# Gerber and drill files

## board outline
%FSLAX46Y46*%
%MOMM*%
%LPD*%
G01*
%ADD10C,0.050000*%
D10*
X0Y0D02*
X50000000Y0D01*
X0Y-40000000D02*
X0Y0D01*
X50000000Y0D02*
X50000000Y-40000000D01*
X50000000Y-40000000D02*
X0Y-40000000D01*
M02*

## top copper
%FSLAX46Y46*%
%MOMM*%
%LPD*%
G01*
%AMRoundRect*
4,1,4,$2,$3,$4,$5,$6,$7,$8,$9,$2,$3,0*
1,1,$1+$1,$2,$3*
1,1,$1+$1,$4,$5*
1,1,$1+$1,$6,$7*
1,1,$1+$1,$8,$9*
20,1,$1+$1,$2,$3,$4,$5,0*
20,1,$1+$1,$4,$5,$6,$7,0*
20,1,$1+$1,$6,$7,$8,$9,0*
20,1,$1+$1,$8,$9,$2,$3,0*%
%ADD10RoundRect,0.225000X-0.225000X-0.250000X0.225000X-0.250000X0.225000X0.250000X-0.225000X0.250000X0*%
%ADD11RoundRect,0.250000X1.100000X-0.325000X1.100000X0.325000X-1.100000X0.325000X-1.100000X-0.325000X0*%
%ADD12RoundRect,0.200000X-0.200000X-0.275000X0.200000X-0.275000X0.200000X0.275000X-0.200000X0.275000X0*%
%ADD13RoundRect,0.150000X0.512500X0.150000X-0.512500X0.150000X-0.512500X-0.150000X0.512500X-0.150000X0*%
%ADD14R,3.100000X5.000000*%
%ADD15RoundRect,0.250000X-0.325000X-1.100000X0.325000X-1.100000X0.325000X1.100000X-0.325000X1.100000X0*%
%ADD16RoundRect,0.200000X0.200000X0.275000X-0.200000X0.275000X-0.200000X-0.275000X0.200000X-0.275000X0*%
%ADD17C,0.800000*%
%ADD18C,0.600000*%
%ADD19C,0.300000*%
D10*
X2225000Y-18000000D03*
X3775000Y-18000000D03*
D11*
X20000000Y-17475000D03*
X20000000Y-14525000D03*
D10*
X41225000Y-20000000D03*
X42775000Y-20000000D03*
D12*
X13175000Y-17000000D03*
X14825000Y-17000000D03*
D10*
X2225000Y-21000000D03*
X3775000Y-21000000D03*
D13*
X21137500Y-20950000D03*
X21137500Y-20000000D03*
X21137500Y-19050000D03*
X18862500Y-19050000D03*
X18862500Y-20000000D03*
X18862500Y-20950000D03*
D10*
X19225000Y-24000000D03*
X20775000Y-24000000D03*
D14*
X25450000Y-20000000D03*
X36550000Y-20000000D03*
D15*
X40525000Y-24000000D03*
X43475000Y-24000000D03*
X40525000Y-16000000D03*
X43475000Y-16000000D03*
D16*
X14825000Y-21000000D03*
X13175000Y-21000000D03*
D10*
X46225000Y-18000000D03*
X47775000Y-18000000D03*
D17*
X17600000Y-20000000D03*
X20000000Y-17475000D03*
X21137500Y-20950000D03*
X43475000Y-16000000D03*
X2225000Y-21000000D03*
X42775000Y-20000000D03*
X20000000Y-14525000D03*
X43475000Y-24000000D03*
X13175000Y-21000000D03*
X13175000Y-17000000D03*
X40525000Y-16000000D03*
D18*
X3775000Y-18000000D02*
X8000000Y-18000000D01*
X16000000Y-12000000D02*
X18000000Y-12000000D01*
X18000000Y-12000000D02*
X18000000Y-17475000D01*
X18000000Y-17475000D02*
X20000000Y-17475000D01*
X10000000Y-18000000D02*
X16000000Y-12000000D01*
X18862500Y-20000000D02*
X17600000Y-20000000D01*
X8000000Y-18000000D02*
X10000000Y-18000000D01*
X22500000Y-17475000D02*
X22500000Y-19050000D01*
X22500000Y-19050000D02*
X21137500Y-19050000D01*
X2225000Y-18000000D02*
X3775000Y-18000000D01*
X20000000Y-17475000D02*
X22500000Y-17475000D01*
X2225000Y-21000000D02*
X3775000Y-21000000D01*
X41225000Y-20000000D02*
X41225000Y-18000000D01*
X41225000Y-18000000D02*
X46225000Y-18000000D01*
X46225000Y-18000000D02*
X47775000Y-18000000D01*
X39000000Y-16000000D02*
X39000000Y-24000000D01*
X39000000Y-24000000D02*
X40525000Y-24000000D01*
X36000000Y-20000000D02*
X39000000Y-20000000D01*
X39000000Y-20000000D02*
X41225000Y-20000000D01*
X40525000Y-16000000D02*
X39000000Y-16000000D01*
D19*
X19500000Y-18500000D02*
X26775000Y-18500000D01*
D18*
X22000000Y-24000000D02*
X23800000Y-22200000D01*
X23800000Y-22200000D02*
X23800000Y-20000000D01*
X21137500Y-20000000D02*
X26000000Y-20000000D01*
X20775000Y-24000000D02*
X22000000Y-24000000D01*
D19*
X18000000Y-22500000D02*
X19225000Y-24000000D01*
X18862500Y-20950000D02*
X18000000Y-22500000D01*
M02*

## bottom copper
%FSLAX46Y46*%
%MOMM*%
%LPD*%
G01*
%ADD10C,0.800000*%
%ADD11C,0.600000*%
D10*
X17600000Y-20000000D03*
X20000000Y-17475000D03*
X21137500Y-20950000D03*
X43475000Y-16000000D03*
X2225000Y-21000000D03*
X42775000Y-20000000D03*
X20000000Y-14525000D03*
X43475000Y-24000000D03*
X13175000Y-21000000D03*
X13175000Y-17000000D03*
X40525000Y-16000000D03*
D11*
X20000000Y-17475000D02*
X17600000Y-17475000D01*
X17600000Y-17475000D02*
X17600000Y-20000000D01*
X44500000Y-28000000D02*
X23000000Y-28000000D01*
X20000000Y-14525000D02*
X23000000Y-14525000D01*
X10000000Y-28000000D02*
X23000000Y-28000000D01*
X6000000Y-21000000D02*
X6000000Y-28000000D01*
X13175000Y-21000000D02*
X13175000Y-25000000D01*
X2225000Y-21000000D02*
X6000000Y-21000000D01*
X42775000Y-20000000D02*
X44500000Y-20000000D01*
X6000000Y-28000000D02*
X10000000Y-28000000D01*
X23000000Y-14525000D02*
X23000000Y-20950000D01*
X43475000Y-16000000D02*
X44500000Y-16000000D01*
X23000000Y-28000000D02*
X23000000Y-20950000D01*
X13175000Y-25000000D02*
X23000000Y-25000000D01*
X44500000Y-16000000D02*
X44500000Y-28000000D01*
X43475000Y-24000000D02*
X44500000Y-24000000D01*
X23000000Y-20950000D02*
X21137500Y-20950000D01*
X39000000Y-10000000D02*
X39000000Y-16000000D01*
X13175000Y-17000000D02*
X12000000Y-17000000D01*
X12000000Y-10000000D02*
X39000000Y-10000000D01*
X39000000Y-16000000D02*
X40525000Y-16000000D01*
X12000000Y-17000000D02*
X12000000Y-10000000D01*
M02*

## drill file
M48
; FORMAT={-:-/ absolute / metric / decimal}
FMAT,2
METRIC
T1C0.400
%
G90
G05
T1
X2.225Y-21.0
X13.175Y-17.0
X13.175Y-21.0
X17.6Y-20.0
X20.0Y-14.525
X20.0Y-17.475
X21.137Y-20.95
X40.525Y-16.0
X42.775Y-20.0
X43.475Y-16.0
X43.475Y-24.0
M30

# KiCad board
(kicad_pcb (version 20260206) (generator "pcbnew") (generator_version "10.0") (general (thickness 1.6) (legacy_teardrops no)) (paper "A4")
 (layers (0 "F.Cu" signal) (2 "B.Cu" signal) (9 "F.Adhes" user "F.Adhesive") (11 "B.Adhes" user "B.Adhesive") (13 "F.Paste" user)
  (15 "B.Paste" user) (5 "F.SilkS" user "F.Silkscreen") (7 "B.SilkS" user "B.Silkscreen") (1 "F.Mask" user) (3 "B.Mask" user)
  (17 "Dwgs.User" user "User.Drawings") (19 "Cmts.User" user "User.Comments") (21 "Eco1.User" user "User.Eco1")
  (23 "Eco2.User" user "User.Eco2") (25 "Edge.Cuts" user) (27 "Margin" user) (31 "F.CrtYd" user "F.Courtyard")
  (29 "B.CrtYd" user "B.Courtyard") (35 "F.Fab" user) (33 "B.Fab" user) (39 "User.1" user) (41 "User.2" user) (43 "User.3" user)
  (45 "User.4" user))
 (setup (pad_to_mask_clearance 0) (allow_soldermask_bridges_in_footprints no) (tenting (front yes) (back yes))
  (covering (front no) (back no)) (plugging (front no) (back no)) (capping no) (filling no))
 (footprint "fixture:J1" (layer "F.Cu") (at 3 18)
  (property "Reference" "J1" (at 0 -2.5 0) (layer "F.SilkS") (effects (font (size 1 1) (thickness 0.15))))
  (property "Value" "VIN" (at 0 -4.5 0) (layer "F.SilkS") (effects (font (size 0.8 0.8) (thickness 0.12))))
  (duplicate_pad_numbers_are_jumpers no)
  (pad "1" smd roundrect (at -0.775 0) (size 0.9 0.95) (layers "F.Cu" "F.Mask" "F.Paste") (roundrect_rratio 0.25) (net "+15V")
   (thermal_bridge_angle 45))
  (pad "2" smd roundrect (at 0.775 0) (size 0.9 0.95) (layers "F.Cu" "F.Mask" "F.Paste") (roundrect_rratio 0.25) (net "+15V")
   (thermal_bridge_angle 45)))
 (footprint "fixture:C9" (layer "F.Cu") (at 20 16 90)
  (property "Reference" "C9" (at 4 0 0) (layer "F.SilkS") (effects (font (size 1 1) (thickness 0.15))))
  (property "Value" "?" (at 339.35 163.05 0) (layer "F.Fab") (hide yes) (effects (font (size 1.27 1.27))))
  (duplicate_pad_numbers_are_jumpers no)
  (pad "1" smd roundrect (at -1.475 0 90) (size 1.15 2.7) (layers "F.Cu" "F.Mask" "F.Paste") (roundrect_rratio 0.217391) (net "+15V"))
  (pad "2" smd roundrect (at 1.475 0 90) (size 1.15 2.7) (layers "F.Cu" "F.Mask" "F.Paste") (roundrect_rratio 0.217391) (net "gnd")))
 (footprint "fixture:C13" (layer "F.Cu") (at 42 20)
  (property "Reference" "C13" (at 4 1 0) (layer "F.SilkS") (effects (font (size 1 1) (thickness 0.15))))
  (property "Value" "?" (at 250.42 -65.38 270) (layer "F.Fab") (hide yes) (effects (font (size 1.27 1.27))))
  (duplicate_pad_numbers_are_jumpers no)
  (pad "1" smd roundrect (at -0.775 0) (size 0.9 0.95) (layers "F.Cu" "F.Mask" "F.Paste") (roundrect_rratio 0.25) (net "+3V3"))
  (pad "2" smd roundrect (at 0.775 0) (size 0.9 0.95) (layers "F.Cu" "F.Mask" "F.Paste") (roundrect_rratio 0.25) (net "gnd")))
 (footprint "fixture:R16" (layer "F.Cu") (at 14 17)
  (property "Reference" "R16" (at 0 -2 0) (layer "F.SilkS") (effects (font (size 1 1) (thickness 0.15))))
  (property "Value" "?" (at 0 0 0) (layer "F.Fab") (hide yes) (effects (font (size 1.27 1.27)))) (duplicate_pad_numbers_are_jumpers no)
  (pad "1" smd roundrect (at -0.825 0) (size 0.8 0.95) (layers "F.Cu" "F.Mask" "F.Paste") (roundrect_rratio 0.25) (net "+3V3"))
  (pad "2" smd roundrect (at 0.825 0) (size 0.8 0.95) (layers "F.Cu" "F.Mask" "F.Paste") (roundrect_rratio 0.25) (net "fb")))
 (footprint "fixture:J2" (layer "F.Cu") (at 3 21)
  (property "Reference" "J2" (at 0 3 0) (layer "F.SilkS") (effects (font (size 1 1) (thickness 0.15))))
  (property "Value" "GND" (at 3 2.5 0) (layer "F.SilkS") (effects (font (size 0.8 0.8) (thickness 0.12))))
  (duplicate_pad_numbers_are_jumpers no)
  (pad "1" smd roundrect (at -0.775 0) (size 0.9 0.95) (layers "F.Cu" "F.Mask" "F.Paste") (roundrect_rratio 0.25) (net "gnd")
   (thermal_bridge_angle 45))
  (pad "2" smd roundrect (at 0.775 0) (size 0.9 0.95) (layers "F.Cu" "F.Mask" "F.Paste") (roundrect_rratio 0.25) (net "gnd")
   (thermal_bridge_angle 45)))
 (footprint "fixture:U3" (layer "F.Cu") (at 20 20 180)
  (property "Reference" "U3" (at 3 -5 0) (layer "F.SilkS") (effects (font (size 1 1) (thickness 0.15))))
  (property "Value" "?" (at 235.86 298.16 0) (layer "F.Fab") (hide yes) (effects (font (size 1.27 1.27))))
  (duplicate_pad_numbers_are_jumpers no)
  (pad "1" smd roundrect (at -1.1375 -0.95 180) (size 1.325 0.6) (layers "F.Cu" "F.Mask" "F.Paste") (roundrect_rratio 0.25) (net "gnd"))
  (pad "2" smd roundrect (at -1.1375 0 180) (size 1.325 0.6) (layers "F.Cu" "F.Mask" "F.Paste") (roundrect_rratio 0.25) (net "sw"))
  (pad "3" smd roundrect (at -1.1375 0.95 180) (size 1.325 0.6) (layers "F.Cu" "F.Mask" "F.Paste") (roundrect_rratio 0.25) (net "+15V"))
  (pad "4" smd roundrect (at 1.1375 0.95 180) (size 1.325 0.6) (layers "F.Cu" "F.Mask" "F.Paste") (roundrect_rratio 0.25) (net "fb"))
  (pad "5" smd roundrect (at 1.1375 0 180) (size 1.325 0.6) (layers "F.Cu" "F.Mask" "F.Paste") (roundrect_rratio 0.25) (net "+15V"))
  (pad "6" smd roundrect (at 1.1375 -0.95 180) (size 1.325 0.6) (layers "F.Cu" "F.Mask" "F.Paste") (roundrect_rratio 0.25) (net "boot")))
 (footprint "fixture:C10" (layer "F.Cu") (at 20 24)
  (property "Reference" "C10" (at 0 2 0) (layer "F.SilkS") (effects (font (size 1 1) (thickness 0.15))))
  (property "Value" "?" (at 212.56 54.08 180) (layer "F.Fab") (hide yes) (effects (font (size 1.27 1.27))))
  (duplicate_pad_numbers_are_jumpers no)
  (pad "1" smd roundrect (at -0.775 0) (size 0.9 0.95) (layers "F.Cu" "F.Mask" "F.Paste") (roundrect_rratio 0.25) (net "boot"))
  (pad "2" smd roundrect (at 0.775 0) (size 0.9 0.95) (layers "F.Cu" "F.Mask" "F.Paste") (roundrect_rratio 0.25) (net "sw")))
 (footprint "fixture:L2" (layer "F.Cu") (at 31 20)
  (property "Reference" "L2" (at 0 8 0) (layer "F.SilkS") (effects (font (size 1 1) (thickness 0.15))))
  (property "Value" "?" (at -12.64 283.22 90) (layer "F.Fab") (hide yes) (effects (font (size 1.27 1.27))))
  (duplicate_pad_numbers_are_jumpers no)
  (pad "1" smd rect (at -5.55 0) (size 3.1 5) (layers "F.Cu" "F.Mask" "F.Paste") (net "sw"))
  (pad "2" smd rect (at 5.55 0) (size 3.1 5) (layers "F.Cu" "F.Mask" "F.Paste") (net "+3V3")))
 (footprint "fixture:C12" (layer "F.Cu") (at 42 24)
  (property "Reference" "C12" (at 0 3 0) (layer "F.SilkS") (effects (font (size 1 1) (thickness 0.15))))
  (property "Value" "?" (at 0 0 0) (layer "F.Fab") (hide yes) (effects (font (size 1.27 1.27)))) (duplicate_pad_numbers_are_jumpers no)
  (pad "1" smd roundrect (at -1.475 0) (size 1.15 2.7) (layers "F.Cu" "F.Mask" "F.Paste") (roundrect_rratio 0.217391) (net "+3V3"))
  (pad "2" smd roundrect (at 1.475 0) (size 1.15 2.7) (layers "F.Cu" "F.Mask" "F.Paste") (roundrect_rratio 0.217391) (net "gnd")))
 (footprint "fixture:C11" (layer "F.Cu") (at 42 16)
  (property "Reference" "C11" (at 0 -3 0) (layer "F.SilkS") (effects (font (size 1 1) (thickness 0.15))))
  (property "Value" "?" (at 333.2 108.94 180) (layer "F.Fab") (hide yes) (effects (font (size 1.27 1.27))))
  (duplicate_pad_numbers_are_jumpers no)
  (pad "1" smd roundrect (at -1.475 0) (size 1.15 2.7) (layers "F.Cu" "F.Mask" "F.Paste") (roundrect_rratio 0.217391) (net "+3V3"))
  (pad "2" smd roundrect (at 1.475 0) (size 1.15 2.7) (layers "F.Cu" "F.Mask" "F.Paste") (roundrect_rratio 0.217391) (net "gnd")))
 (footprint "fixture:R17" (layer "F.Cu") (at 14 21 180)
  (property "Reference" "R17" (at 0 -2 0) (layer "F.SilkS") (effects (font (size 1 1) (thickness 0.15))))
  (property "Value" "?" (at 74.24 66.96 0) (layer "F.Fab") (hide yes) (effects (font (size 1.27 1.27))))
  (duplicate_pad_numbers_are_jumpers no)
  (pad "1" smd roundrect (at -0.825 0 180) (size 0.8 0.95) (layers "F.Cu" "F.Mask" "F.Paste") (roundrect_rratio 0.25) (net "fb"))
  (pad "2" smd roundrect (at 0.825 0 180) (size 0.8 0.95) (layers "F.Cu" "F.Mask" "F.Paste") (roundrect_rratio 0.25) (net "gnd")))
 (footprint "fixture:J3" (layer "F.Cu") (at 47 18)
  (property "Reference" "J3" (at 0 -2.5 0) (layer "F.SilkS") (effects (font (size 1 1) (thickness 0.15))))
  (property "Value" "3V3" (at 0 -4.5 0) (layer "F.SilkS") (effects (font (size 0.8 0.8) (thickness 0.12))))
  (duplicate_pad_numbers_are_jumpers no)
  (pad "1" smd roundrect (at -0.775 0) (size 0.9 0.95) (layers "F.Cu" "F.Mask" "F.Paste") (roundrect_rratio 0.25) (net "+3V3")
   (thermal_bridge_angle 45))
  (pad "2" smd roundrect (at 0.775 0) (size 0.9 0.95) (layers "F.Cu" "F.Mask" "F.Paste") (roundrect_rratio 0.25) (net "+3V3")
   (thermal_bridge_angle 45)))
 (gr_line (start 0 0) (end 50 0) (stroke (width 0.05) (type default)) (layer "Edge.Cuts"))
 (gr_line (start 0 40) (end 0 0) (stroke (width 0.05) (type default)) (layer "Edge.Cuts"))
 (gr_line (start 50 0) (end 50 40) (stroke (width 0.05) (type default)) (layer "Edge.Cuts"))
 (gr_line (start 50 40) (end 0 40) (stroke (width 0.05) (type default)) (layer "Edge.Cuts"))
 (segment (start 3.775 18) (end 8 18) (width 0.6) (layer "F.Cu") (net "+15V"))
 (segment (start 16 12) (end 18 12) (width 0.6) (layer "F.Cu") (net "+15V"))
 (segment (start 18 12) (end 18 17.475) (width 0.6) (layer "F.Cu") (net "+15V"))
 (segment (start 18 17.475) (end 20 17.475) (width 0.6) (layer "F.Cu") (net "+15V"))
 (segment (start 10 18) (end 16 12) (width 0.6) (layer "F.Cu") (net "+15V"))
 (segment (start 18.8625 20) (end 17.6 20) (width 0.6) (layer "F.Cu") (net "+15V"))
 (segment (start 8 18) (end 10 18) (width 0.6) (layer "F.Cu") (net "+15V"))
 (segment (start 22.5 17.475) (end 22.5 19.05) (width 0.6) (layer "F.Cu") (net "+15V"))
 (segment (start 22.5 19.05) (end 21.1375 19.05) (width 0.6) (layer "F.Cu") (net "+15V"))
 (segment (start 2.225 18) (end 3.775 18) (width 0.6) (layer "F.Cu") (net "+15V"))
 (segment (start 20 17.475) (end 22.5 17.475) (width 0.6) (layer "F.Cu") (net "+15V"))
 (via (at 17.6 20) (size 0.8) (drill 0.4) (layers "F.Cu" "B.Cu") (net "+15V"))
 (via (at 20 17.475) (size 0.8) (drill 0.4) (layers "F.Cu" "B.Cu") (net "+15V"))
 (segment (start 20 17.475) (end 17.6 17.475) (width 0.6) (layer "B.Cu") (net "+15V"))
 (segment (start 17.6 17.475) (end 17.6 20) (width 0.6) (layer "B.Cu") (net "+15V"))
 (segment (start 2.225 21) (end 3.775 21) (width 0.6) (layer "F.Cu") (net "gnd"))
 (via (at 21.1375 20.95) (size 0.8) (drill 0.4) (layers "F.Cu" "B.Cu") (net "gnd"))
 (via (at 43.475 16) (size 0.8) (drill 0.4) (layers "F.Cu" "B.Cu") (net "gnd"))
 (via (at 2.225 21) (size 0.8) (drill 0.4) (layers "F.Cu" "B.Cu") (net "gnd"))
 (via (at 42.775 20) (size 0.8) (drill 0.4) (layers "F.Cu" "B.Cu") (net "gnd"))
 (via (at 20 14.525) (size 0.8) (drill 0.4) (layers "F.Cu" "B.Cu") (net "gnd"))
 (via (at 43.475 24) (size 0.8) (drill 0.4) (layers "F.Cu" "B.Cu") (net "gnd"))
 (via (at 13.175 21) (size 0.8) (drill 0.4) (layers "F.Cu" "B.Cu") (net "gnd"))
 (segment (start 44.5 28) (end 23 28) (width 0.6) (layer "B.Cu") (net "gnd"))
 (segment (start 20 14.525) (end 23 14.525) (width 0.6) (layer "B.Cu") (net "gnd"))
 (segment (start 10 28) (end 23 28) (width 0.6) (layer "B.Cu") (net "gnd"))
 (segment (start 6 21) (end 6 28) (width 0.6) (layer "B.Cu") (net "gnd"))
 (segment (start 13.175 21) (end 13.175 25) (width 0.6) (layer "B.Cu") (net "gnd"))
 (segment (start 2.225 21) (end 6 21) (width 0.6) (layer "B.Cu") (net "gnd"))
 (segment (start 42.775 20) (end 44.5 20) (width 0.6) (layer "B.Cu") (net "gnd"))
 (segment (start 6 28) (end 10 28) (width 0.6) (layer "B.Cu") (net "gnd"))
 (segment (start 23 14.525) (end 23 20.95) (width 0.6) (layer "B.Cu") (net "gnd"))
 (segment (start 43.475 16) (end 44.5 16) (width 0.6) (layer "B.Cu") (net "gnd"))
 (segment (start 23 28) (end 23 20.95) (width 0.6) (layer "B.Cu") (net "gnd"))
 (segment (start 13.175 25) (end 23 25) (width 0.6) (layer "B.Cu") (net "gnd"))
 (segment (start 44.5 16) (end 44.5 28) (width 0.6) (layer "B.Cu") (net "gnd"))
 (segment (start 43.475 24) (end 44.5 24) (width 0.6) (layer "B.Cu") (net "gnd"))
 (segment (start 23 20.95) (end 21.1375 20.95) (width 0.6) (layer "B.Cu") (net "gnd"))
 (segment (start 41.225 20) (end 41.225 18) (width 0.6) (layer "F.Cu") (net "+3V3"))
 (segment (start 41.225 18) (end 46.225 18) (width 0.6) (layer "F.Cu") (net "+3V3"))
 (segment (start 46.225 18) (end 47.775 18) (width 0.6) (layer "F.Cu") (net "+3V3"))
 (segment (start 39 16) (end 39 24) (width 0.6) (layer "F.Cu") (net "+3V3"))
 (segment (start 39 24) (end 40.525 24) (width 0.6) (layer "F.Cu") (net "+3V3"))
 (segment (start 36 20) (end 39 20) (width 0.6) (layer "F.Cu") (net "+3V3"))
 (segment (start 39 20) (end 41.225 20) (width 0.6) (layer "F.Cu") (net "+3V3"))
 (segment (start 40.525 16) (end 39 16) (width 0.6) (layer "F.Cu") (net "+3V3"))
 (via (at 13.175 17) (size 0.8) (drill 0.4) (layers "F.Cu" "B.Cu") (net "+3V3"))
 (via (at 40.525 16) (size 0.8) (drill 0.4) (layers "F.Cu" "B.Cu") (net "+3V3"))
 (segment (start 39 10) (end 39 16) (width 0.6) (layer "B.Cu") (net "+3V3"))
 (segment (start 13.175 17) (end 12 17) (width 0.6) (layer "B.Cu") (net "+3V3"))
 (segment (start 12 10) (end 39 10) (width 0.6) (layer "B.Cu") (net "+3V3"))
 (segment (start 39 16) (end 40.525 16) (width 0.6) (layer "B.Cu") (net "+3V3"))
 (segment (start 12 17) (end 12 10) (width 0.6) (layer "B.Cu") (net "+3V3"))
 (segment (start 19.5 18.5) (end 26.775 18.5) (width 0.3) (layer "F.Cu") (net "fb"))
 (segment (start 22 24) (end 23.8 22.2) (width 0.6) (layer "F.Cu") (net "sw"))
 (segment (start 23.8 22.2) (end 23.8 20) (width 0.6) (layer "F.Cu") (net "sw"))
 (segment (start 21.1375 20) (end 26 20) (width 0.6) (layer "F.Cu") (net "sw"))
 (segment (start 20.775 24) (end 22 24) (width 0.6) (layer "F.Cu") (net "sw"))
 (segment (start 18 22.5) (end 19.225 24) (width 0.3) (layer "F.Cu") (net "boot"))
 (segment (start 18.8625 20.95) (end 18 22.5) (width 0.3) (layer "F.Cu") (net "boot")))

